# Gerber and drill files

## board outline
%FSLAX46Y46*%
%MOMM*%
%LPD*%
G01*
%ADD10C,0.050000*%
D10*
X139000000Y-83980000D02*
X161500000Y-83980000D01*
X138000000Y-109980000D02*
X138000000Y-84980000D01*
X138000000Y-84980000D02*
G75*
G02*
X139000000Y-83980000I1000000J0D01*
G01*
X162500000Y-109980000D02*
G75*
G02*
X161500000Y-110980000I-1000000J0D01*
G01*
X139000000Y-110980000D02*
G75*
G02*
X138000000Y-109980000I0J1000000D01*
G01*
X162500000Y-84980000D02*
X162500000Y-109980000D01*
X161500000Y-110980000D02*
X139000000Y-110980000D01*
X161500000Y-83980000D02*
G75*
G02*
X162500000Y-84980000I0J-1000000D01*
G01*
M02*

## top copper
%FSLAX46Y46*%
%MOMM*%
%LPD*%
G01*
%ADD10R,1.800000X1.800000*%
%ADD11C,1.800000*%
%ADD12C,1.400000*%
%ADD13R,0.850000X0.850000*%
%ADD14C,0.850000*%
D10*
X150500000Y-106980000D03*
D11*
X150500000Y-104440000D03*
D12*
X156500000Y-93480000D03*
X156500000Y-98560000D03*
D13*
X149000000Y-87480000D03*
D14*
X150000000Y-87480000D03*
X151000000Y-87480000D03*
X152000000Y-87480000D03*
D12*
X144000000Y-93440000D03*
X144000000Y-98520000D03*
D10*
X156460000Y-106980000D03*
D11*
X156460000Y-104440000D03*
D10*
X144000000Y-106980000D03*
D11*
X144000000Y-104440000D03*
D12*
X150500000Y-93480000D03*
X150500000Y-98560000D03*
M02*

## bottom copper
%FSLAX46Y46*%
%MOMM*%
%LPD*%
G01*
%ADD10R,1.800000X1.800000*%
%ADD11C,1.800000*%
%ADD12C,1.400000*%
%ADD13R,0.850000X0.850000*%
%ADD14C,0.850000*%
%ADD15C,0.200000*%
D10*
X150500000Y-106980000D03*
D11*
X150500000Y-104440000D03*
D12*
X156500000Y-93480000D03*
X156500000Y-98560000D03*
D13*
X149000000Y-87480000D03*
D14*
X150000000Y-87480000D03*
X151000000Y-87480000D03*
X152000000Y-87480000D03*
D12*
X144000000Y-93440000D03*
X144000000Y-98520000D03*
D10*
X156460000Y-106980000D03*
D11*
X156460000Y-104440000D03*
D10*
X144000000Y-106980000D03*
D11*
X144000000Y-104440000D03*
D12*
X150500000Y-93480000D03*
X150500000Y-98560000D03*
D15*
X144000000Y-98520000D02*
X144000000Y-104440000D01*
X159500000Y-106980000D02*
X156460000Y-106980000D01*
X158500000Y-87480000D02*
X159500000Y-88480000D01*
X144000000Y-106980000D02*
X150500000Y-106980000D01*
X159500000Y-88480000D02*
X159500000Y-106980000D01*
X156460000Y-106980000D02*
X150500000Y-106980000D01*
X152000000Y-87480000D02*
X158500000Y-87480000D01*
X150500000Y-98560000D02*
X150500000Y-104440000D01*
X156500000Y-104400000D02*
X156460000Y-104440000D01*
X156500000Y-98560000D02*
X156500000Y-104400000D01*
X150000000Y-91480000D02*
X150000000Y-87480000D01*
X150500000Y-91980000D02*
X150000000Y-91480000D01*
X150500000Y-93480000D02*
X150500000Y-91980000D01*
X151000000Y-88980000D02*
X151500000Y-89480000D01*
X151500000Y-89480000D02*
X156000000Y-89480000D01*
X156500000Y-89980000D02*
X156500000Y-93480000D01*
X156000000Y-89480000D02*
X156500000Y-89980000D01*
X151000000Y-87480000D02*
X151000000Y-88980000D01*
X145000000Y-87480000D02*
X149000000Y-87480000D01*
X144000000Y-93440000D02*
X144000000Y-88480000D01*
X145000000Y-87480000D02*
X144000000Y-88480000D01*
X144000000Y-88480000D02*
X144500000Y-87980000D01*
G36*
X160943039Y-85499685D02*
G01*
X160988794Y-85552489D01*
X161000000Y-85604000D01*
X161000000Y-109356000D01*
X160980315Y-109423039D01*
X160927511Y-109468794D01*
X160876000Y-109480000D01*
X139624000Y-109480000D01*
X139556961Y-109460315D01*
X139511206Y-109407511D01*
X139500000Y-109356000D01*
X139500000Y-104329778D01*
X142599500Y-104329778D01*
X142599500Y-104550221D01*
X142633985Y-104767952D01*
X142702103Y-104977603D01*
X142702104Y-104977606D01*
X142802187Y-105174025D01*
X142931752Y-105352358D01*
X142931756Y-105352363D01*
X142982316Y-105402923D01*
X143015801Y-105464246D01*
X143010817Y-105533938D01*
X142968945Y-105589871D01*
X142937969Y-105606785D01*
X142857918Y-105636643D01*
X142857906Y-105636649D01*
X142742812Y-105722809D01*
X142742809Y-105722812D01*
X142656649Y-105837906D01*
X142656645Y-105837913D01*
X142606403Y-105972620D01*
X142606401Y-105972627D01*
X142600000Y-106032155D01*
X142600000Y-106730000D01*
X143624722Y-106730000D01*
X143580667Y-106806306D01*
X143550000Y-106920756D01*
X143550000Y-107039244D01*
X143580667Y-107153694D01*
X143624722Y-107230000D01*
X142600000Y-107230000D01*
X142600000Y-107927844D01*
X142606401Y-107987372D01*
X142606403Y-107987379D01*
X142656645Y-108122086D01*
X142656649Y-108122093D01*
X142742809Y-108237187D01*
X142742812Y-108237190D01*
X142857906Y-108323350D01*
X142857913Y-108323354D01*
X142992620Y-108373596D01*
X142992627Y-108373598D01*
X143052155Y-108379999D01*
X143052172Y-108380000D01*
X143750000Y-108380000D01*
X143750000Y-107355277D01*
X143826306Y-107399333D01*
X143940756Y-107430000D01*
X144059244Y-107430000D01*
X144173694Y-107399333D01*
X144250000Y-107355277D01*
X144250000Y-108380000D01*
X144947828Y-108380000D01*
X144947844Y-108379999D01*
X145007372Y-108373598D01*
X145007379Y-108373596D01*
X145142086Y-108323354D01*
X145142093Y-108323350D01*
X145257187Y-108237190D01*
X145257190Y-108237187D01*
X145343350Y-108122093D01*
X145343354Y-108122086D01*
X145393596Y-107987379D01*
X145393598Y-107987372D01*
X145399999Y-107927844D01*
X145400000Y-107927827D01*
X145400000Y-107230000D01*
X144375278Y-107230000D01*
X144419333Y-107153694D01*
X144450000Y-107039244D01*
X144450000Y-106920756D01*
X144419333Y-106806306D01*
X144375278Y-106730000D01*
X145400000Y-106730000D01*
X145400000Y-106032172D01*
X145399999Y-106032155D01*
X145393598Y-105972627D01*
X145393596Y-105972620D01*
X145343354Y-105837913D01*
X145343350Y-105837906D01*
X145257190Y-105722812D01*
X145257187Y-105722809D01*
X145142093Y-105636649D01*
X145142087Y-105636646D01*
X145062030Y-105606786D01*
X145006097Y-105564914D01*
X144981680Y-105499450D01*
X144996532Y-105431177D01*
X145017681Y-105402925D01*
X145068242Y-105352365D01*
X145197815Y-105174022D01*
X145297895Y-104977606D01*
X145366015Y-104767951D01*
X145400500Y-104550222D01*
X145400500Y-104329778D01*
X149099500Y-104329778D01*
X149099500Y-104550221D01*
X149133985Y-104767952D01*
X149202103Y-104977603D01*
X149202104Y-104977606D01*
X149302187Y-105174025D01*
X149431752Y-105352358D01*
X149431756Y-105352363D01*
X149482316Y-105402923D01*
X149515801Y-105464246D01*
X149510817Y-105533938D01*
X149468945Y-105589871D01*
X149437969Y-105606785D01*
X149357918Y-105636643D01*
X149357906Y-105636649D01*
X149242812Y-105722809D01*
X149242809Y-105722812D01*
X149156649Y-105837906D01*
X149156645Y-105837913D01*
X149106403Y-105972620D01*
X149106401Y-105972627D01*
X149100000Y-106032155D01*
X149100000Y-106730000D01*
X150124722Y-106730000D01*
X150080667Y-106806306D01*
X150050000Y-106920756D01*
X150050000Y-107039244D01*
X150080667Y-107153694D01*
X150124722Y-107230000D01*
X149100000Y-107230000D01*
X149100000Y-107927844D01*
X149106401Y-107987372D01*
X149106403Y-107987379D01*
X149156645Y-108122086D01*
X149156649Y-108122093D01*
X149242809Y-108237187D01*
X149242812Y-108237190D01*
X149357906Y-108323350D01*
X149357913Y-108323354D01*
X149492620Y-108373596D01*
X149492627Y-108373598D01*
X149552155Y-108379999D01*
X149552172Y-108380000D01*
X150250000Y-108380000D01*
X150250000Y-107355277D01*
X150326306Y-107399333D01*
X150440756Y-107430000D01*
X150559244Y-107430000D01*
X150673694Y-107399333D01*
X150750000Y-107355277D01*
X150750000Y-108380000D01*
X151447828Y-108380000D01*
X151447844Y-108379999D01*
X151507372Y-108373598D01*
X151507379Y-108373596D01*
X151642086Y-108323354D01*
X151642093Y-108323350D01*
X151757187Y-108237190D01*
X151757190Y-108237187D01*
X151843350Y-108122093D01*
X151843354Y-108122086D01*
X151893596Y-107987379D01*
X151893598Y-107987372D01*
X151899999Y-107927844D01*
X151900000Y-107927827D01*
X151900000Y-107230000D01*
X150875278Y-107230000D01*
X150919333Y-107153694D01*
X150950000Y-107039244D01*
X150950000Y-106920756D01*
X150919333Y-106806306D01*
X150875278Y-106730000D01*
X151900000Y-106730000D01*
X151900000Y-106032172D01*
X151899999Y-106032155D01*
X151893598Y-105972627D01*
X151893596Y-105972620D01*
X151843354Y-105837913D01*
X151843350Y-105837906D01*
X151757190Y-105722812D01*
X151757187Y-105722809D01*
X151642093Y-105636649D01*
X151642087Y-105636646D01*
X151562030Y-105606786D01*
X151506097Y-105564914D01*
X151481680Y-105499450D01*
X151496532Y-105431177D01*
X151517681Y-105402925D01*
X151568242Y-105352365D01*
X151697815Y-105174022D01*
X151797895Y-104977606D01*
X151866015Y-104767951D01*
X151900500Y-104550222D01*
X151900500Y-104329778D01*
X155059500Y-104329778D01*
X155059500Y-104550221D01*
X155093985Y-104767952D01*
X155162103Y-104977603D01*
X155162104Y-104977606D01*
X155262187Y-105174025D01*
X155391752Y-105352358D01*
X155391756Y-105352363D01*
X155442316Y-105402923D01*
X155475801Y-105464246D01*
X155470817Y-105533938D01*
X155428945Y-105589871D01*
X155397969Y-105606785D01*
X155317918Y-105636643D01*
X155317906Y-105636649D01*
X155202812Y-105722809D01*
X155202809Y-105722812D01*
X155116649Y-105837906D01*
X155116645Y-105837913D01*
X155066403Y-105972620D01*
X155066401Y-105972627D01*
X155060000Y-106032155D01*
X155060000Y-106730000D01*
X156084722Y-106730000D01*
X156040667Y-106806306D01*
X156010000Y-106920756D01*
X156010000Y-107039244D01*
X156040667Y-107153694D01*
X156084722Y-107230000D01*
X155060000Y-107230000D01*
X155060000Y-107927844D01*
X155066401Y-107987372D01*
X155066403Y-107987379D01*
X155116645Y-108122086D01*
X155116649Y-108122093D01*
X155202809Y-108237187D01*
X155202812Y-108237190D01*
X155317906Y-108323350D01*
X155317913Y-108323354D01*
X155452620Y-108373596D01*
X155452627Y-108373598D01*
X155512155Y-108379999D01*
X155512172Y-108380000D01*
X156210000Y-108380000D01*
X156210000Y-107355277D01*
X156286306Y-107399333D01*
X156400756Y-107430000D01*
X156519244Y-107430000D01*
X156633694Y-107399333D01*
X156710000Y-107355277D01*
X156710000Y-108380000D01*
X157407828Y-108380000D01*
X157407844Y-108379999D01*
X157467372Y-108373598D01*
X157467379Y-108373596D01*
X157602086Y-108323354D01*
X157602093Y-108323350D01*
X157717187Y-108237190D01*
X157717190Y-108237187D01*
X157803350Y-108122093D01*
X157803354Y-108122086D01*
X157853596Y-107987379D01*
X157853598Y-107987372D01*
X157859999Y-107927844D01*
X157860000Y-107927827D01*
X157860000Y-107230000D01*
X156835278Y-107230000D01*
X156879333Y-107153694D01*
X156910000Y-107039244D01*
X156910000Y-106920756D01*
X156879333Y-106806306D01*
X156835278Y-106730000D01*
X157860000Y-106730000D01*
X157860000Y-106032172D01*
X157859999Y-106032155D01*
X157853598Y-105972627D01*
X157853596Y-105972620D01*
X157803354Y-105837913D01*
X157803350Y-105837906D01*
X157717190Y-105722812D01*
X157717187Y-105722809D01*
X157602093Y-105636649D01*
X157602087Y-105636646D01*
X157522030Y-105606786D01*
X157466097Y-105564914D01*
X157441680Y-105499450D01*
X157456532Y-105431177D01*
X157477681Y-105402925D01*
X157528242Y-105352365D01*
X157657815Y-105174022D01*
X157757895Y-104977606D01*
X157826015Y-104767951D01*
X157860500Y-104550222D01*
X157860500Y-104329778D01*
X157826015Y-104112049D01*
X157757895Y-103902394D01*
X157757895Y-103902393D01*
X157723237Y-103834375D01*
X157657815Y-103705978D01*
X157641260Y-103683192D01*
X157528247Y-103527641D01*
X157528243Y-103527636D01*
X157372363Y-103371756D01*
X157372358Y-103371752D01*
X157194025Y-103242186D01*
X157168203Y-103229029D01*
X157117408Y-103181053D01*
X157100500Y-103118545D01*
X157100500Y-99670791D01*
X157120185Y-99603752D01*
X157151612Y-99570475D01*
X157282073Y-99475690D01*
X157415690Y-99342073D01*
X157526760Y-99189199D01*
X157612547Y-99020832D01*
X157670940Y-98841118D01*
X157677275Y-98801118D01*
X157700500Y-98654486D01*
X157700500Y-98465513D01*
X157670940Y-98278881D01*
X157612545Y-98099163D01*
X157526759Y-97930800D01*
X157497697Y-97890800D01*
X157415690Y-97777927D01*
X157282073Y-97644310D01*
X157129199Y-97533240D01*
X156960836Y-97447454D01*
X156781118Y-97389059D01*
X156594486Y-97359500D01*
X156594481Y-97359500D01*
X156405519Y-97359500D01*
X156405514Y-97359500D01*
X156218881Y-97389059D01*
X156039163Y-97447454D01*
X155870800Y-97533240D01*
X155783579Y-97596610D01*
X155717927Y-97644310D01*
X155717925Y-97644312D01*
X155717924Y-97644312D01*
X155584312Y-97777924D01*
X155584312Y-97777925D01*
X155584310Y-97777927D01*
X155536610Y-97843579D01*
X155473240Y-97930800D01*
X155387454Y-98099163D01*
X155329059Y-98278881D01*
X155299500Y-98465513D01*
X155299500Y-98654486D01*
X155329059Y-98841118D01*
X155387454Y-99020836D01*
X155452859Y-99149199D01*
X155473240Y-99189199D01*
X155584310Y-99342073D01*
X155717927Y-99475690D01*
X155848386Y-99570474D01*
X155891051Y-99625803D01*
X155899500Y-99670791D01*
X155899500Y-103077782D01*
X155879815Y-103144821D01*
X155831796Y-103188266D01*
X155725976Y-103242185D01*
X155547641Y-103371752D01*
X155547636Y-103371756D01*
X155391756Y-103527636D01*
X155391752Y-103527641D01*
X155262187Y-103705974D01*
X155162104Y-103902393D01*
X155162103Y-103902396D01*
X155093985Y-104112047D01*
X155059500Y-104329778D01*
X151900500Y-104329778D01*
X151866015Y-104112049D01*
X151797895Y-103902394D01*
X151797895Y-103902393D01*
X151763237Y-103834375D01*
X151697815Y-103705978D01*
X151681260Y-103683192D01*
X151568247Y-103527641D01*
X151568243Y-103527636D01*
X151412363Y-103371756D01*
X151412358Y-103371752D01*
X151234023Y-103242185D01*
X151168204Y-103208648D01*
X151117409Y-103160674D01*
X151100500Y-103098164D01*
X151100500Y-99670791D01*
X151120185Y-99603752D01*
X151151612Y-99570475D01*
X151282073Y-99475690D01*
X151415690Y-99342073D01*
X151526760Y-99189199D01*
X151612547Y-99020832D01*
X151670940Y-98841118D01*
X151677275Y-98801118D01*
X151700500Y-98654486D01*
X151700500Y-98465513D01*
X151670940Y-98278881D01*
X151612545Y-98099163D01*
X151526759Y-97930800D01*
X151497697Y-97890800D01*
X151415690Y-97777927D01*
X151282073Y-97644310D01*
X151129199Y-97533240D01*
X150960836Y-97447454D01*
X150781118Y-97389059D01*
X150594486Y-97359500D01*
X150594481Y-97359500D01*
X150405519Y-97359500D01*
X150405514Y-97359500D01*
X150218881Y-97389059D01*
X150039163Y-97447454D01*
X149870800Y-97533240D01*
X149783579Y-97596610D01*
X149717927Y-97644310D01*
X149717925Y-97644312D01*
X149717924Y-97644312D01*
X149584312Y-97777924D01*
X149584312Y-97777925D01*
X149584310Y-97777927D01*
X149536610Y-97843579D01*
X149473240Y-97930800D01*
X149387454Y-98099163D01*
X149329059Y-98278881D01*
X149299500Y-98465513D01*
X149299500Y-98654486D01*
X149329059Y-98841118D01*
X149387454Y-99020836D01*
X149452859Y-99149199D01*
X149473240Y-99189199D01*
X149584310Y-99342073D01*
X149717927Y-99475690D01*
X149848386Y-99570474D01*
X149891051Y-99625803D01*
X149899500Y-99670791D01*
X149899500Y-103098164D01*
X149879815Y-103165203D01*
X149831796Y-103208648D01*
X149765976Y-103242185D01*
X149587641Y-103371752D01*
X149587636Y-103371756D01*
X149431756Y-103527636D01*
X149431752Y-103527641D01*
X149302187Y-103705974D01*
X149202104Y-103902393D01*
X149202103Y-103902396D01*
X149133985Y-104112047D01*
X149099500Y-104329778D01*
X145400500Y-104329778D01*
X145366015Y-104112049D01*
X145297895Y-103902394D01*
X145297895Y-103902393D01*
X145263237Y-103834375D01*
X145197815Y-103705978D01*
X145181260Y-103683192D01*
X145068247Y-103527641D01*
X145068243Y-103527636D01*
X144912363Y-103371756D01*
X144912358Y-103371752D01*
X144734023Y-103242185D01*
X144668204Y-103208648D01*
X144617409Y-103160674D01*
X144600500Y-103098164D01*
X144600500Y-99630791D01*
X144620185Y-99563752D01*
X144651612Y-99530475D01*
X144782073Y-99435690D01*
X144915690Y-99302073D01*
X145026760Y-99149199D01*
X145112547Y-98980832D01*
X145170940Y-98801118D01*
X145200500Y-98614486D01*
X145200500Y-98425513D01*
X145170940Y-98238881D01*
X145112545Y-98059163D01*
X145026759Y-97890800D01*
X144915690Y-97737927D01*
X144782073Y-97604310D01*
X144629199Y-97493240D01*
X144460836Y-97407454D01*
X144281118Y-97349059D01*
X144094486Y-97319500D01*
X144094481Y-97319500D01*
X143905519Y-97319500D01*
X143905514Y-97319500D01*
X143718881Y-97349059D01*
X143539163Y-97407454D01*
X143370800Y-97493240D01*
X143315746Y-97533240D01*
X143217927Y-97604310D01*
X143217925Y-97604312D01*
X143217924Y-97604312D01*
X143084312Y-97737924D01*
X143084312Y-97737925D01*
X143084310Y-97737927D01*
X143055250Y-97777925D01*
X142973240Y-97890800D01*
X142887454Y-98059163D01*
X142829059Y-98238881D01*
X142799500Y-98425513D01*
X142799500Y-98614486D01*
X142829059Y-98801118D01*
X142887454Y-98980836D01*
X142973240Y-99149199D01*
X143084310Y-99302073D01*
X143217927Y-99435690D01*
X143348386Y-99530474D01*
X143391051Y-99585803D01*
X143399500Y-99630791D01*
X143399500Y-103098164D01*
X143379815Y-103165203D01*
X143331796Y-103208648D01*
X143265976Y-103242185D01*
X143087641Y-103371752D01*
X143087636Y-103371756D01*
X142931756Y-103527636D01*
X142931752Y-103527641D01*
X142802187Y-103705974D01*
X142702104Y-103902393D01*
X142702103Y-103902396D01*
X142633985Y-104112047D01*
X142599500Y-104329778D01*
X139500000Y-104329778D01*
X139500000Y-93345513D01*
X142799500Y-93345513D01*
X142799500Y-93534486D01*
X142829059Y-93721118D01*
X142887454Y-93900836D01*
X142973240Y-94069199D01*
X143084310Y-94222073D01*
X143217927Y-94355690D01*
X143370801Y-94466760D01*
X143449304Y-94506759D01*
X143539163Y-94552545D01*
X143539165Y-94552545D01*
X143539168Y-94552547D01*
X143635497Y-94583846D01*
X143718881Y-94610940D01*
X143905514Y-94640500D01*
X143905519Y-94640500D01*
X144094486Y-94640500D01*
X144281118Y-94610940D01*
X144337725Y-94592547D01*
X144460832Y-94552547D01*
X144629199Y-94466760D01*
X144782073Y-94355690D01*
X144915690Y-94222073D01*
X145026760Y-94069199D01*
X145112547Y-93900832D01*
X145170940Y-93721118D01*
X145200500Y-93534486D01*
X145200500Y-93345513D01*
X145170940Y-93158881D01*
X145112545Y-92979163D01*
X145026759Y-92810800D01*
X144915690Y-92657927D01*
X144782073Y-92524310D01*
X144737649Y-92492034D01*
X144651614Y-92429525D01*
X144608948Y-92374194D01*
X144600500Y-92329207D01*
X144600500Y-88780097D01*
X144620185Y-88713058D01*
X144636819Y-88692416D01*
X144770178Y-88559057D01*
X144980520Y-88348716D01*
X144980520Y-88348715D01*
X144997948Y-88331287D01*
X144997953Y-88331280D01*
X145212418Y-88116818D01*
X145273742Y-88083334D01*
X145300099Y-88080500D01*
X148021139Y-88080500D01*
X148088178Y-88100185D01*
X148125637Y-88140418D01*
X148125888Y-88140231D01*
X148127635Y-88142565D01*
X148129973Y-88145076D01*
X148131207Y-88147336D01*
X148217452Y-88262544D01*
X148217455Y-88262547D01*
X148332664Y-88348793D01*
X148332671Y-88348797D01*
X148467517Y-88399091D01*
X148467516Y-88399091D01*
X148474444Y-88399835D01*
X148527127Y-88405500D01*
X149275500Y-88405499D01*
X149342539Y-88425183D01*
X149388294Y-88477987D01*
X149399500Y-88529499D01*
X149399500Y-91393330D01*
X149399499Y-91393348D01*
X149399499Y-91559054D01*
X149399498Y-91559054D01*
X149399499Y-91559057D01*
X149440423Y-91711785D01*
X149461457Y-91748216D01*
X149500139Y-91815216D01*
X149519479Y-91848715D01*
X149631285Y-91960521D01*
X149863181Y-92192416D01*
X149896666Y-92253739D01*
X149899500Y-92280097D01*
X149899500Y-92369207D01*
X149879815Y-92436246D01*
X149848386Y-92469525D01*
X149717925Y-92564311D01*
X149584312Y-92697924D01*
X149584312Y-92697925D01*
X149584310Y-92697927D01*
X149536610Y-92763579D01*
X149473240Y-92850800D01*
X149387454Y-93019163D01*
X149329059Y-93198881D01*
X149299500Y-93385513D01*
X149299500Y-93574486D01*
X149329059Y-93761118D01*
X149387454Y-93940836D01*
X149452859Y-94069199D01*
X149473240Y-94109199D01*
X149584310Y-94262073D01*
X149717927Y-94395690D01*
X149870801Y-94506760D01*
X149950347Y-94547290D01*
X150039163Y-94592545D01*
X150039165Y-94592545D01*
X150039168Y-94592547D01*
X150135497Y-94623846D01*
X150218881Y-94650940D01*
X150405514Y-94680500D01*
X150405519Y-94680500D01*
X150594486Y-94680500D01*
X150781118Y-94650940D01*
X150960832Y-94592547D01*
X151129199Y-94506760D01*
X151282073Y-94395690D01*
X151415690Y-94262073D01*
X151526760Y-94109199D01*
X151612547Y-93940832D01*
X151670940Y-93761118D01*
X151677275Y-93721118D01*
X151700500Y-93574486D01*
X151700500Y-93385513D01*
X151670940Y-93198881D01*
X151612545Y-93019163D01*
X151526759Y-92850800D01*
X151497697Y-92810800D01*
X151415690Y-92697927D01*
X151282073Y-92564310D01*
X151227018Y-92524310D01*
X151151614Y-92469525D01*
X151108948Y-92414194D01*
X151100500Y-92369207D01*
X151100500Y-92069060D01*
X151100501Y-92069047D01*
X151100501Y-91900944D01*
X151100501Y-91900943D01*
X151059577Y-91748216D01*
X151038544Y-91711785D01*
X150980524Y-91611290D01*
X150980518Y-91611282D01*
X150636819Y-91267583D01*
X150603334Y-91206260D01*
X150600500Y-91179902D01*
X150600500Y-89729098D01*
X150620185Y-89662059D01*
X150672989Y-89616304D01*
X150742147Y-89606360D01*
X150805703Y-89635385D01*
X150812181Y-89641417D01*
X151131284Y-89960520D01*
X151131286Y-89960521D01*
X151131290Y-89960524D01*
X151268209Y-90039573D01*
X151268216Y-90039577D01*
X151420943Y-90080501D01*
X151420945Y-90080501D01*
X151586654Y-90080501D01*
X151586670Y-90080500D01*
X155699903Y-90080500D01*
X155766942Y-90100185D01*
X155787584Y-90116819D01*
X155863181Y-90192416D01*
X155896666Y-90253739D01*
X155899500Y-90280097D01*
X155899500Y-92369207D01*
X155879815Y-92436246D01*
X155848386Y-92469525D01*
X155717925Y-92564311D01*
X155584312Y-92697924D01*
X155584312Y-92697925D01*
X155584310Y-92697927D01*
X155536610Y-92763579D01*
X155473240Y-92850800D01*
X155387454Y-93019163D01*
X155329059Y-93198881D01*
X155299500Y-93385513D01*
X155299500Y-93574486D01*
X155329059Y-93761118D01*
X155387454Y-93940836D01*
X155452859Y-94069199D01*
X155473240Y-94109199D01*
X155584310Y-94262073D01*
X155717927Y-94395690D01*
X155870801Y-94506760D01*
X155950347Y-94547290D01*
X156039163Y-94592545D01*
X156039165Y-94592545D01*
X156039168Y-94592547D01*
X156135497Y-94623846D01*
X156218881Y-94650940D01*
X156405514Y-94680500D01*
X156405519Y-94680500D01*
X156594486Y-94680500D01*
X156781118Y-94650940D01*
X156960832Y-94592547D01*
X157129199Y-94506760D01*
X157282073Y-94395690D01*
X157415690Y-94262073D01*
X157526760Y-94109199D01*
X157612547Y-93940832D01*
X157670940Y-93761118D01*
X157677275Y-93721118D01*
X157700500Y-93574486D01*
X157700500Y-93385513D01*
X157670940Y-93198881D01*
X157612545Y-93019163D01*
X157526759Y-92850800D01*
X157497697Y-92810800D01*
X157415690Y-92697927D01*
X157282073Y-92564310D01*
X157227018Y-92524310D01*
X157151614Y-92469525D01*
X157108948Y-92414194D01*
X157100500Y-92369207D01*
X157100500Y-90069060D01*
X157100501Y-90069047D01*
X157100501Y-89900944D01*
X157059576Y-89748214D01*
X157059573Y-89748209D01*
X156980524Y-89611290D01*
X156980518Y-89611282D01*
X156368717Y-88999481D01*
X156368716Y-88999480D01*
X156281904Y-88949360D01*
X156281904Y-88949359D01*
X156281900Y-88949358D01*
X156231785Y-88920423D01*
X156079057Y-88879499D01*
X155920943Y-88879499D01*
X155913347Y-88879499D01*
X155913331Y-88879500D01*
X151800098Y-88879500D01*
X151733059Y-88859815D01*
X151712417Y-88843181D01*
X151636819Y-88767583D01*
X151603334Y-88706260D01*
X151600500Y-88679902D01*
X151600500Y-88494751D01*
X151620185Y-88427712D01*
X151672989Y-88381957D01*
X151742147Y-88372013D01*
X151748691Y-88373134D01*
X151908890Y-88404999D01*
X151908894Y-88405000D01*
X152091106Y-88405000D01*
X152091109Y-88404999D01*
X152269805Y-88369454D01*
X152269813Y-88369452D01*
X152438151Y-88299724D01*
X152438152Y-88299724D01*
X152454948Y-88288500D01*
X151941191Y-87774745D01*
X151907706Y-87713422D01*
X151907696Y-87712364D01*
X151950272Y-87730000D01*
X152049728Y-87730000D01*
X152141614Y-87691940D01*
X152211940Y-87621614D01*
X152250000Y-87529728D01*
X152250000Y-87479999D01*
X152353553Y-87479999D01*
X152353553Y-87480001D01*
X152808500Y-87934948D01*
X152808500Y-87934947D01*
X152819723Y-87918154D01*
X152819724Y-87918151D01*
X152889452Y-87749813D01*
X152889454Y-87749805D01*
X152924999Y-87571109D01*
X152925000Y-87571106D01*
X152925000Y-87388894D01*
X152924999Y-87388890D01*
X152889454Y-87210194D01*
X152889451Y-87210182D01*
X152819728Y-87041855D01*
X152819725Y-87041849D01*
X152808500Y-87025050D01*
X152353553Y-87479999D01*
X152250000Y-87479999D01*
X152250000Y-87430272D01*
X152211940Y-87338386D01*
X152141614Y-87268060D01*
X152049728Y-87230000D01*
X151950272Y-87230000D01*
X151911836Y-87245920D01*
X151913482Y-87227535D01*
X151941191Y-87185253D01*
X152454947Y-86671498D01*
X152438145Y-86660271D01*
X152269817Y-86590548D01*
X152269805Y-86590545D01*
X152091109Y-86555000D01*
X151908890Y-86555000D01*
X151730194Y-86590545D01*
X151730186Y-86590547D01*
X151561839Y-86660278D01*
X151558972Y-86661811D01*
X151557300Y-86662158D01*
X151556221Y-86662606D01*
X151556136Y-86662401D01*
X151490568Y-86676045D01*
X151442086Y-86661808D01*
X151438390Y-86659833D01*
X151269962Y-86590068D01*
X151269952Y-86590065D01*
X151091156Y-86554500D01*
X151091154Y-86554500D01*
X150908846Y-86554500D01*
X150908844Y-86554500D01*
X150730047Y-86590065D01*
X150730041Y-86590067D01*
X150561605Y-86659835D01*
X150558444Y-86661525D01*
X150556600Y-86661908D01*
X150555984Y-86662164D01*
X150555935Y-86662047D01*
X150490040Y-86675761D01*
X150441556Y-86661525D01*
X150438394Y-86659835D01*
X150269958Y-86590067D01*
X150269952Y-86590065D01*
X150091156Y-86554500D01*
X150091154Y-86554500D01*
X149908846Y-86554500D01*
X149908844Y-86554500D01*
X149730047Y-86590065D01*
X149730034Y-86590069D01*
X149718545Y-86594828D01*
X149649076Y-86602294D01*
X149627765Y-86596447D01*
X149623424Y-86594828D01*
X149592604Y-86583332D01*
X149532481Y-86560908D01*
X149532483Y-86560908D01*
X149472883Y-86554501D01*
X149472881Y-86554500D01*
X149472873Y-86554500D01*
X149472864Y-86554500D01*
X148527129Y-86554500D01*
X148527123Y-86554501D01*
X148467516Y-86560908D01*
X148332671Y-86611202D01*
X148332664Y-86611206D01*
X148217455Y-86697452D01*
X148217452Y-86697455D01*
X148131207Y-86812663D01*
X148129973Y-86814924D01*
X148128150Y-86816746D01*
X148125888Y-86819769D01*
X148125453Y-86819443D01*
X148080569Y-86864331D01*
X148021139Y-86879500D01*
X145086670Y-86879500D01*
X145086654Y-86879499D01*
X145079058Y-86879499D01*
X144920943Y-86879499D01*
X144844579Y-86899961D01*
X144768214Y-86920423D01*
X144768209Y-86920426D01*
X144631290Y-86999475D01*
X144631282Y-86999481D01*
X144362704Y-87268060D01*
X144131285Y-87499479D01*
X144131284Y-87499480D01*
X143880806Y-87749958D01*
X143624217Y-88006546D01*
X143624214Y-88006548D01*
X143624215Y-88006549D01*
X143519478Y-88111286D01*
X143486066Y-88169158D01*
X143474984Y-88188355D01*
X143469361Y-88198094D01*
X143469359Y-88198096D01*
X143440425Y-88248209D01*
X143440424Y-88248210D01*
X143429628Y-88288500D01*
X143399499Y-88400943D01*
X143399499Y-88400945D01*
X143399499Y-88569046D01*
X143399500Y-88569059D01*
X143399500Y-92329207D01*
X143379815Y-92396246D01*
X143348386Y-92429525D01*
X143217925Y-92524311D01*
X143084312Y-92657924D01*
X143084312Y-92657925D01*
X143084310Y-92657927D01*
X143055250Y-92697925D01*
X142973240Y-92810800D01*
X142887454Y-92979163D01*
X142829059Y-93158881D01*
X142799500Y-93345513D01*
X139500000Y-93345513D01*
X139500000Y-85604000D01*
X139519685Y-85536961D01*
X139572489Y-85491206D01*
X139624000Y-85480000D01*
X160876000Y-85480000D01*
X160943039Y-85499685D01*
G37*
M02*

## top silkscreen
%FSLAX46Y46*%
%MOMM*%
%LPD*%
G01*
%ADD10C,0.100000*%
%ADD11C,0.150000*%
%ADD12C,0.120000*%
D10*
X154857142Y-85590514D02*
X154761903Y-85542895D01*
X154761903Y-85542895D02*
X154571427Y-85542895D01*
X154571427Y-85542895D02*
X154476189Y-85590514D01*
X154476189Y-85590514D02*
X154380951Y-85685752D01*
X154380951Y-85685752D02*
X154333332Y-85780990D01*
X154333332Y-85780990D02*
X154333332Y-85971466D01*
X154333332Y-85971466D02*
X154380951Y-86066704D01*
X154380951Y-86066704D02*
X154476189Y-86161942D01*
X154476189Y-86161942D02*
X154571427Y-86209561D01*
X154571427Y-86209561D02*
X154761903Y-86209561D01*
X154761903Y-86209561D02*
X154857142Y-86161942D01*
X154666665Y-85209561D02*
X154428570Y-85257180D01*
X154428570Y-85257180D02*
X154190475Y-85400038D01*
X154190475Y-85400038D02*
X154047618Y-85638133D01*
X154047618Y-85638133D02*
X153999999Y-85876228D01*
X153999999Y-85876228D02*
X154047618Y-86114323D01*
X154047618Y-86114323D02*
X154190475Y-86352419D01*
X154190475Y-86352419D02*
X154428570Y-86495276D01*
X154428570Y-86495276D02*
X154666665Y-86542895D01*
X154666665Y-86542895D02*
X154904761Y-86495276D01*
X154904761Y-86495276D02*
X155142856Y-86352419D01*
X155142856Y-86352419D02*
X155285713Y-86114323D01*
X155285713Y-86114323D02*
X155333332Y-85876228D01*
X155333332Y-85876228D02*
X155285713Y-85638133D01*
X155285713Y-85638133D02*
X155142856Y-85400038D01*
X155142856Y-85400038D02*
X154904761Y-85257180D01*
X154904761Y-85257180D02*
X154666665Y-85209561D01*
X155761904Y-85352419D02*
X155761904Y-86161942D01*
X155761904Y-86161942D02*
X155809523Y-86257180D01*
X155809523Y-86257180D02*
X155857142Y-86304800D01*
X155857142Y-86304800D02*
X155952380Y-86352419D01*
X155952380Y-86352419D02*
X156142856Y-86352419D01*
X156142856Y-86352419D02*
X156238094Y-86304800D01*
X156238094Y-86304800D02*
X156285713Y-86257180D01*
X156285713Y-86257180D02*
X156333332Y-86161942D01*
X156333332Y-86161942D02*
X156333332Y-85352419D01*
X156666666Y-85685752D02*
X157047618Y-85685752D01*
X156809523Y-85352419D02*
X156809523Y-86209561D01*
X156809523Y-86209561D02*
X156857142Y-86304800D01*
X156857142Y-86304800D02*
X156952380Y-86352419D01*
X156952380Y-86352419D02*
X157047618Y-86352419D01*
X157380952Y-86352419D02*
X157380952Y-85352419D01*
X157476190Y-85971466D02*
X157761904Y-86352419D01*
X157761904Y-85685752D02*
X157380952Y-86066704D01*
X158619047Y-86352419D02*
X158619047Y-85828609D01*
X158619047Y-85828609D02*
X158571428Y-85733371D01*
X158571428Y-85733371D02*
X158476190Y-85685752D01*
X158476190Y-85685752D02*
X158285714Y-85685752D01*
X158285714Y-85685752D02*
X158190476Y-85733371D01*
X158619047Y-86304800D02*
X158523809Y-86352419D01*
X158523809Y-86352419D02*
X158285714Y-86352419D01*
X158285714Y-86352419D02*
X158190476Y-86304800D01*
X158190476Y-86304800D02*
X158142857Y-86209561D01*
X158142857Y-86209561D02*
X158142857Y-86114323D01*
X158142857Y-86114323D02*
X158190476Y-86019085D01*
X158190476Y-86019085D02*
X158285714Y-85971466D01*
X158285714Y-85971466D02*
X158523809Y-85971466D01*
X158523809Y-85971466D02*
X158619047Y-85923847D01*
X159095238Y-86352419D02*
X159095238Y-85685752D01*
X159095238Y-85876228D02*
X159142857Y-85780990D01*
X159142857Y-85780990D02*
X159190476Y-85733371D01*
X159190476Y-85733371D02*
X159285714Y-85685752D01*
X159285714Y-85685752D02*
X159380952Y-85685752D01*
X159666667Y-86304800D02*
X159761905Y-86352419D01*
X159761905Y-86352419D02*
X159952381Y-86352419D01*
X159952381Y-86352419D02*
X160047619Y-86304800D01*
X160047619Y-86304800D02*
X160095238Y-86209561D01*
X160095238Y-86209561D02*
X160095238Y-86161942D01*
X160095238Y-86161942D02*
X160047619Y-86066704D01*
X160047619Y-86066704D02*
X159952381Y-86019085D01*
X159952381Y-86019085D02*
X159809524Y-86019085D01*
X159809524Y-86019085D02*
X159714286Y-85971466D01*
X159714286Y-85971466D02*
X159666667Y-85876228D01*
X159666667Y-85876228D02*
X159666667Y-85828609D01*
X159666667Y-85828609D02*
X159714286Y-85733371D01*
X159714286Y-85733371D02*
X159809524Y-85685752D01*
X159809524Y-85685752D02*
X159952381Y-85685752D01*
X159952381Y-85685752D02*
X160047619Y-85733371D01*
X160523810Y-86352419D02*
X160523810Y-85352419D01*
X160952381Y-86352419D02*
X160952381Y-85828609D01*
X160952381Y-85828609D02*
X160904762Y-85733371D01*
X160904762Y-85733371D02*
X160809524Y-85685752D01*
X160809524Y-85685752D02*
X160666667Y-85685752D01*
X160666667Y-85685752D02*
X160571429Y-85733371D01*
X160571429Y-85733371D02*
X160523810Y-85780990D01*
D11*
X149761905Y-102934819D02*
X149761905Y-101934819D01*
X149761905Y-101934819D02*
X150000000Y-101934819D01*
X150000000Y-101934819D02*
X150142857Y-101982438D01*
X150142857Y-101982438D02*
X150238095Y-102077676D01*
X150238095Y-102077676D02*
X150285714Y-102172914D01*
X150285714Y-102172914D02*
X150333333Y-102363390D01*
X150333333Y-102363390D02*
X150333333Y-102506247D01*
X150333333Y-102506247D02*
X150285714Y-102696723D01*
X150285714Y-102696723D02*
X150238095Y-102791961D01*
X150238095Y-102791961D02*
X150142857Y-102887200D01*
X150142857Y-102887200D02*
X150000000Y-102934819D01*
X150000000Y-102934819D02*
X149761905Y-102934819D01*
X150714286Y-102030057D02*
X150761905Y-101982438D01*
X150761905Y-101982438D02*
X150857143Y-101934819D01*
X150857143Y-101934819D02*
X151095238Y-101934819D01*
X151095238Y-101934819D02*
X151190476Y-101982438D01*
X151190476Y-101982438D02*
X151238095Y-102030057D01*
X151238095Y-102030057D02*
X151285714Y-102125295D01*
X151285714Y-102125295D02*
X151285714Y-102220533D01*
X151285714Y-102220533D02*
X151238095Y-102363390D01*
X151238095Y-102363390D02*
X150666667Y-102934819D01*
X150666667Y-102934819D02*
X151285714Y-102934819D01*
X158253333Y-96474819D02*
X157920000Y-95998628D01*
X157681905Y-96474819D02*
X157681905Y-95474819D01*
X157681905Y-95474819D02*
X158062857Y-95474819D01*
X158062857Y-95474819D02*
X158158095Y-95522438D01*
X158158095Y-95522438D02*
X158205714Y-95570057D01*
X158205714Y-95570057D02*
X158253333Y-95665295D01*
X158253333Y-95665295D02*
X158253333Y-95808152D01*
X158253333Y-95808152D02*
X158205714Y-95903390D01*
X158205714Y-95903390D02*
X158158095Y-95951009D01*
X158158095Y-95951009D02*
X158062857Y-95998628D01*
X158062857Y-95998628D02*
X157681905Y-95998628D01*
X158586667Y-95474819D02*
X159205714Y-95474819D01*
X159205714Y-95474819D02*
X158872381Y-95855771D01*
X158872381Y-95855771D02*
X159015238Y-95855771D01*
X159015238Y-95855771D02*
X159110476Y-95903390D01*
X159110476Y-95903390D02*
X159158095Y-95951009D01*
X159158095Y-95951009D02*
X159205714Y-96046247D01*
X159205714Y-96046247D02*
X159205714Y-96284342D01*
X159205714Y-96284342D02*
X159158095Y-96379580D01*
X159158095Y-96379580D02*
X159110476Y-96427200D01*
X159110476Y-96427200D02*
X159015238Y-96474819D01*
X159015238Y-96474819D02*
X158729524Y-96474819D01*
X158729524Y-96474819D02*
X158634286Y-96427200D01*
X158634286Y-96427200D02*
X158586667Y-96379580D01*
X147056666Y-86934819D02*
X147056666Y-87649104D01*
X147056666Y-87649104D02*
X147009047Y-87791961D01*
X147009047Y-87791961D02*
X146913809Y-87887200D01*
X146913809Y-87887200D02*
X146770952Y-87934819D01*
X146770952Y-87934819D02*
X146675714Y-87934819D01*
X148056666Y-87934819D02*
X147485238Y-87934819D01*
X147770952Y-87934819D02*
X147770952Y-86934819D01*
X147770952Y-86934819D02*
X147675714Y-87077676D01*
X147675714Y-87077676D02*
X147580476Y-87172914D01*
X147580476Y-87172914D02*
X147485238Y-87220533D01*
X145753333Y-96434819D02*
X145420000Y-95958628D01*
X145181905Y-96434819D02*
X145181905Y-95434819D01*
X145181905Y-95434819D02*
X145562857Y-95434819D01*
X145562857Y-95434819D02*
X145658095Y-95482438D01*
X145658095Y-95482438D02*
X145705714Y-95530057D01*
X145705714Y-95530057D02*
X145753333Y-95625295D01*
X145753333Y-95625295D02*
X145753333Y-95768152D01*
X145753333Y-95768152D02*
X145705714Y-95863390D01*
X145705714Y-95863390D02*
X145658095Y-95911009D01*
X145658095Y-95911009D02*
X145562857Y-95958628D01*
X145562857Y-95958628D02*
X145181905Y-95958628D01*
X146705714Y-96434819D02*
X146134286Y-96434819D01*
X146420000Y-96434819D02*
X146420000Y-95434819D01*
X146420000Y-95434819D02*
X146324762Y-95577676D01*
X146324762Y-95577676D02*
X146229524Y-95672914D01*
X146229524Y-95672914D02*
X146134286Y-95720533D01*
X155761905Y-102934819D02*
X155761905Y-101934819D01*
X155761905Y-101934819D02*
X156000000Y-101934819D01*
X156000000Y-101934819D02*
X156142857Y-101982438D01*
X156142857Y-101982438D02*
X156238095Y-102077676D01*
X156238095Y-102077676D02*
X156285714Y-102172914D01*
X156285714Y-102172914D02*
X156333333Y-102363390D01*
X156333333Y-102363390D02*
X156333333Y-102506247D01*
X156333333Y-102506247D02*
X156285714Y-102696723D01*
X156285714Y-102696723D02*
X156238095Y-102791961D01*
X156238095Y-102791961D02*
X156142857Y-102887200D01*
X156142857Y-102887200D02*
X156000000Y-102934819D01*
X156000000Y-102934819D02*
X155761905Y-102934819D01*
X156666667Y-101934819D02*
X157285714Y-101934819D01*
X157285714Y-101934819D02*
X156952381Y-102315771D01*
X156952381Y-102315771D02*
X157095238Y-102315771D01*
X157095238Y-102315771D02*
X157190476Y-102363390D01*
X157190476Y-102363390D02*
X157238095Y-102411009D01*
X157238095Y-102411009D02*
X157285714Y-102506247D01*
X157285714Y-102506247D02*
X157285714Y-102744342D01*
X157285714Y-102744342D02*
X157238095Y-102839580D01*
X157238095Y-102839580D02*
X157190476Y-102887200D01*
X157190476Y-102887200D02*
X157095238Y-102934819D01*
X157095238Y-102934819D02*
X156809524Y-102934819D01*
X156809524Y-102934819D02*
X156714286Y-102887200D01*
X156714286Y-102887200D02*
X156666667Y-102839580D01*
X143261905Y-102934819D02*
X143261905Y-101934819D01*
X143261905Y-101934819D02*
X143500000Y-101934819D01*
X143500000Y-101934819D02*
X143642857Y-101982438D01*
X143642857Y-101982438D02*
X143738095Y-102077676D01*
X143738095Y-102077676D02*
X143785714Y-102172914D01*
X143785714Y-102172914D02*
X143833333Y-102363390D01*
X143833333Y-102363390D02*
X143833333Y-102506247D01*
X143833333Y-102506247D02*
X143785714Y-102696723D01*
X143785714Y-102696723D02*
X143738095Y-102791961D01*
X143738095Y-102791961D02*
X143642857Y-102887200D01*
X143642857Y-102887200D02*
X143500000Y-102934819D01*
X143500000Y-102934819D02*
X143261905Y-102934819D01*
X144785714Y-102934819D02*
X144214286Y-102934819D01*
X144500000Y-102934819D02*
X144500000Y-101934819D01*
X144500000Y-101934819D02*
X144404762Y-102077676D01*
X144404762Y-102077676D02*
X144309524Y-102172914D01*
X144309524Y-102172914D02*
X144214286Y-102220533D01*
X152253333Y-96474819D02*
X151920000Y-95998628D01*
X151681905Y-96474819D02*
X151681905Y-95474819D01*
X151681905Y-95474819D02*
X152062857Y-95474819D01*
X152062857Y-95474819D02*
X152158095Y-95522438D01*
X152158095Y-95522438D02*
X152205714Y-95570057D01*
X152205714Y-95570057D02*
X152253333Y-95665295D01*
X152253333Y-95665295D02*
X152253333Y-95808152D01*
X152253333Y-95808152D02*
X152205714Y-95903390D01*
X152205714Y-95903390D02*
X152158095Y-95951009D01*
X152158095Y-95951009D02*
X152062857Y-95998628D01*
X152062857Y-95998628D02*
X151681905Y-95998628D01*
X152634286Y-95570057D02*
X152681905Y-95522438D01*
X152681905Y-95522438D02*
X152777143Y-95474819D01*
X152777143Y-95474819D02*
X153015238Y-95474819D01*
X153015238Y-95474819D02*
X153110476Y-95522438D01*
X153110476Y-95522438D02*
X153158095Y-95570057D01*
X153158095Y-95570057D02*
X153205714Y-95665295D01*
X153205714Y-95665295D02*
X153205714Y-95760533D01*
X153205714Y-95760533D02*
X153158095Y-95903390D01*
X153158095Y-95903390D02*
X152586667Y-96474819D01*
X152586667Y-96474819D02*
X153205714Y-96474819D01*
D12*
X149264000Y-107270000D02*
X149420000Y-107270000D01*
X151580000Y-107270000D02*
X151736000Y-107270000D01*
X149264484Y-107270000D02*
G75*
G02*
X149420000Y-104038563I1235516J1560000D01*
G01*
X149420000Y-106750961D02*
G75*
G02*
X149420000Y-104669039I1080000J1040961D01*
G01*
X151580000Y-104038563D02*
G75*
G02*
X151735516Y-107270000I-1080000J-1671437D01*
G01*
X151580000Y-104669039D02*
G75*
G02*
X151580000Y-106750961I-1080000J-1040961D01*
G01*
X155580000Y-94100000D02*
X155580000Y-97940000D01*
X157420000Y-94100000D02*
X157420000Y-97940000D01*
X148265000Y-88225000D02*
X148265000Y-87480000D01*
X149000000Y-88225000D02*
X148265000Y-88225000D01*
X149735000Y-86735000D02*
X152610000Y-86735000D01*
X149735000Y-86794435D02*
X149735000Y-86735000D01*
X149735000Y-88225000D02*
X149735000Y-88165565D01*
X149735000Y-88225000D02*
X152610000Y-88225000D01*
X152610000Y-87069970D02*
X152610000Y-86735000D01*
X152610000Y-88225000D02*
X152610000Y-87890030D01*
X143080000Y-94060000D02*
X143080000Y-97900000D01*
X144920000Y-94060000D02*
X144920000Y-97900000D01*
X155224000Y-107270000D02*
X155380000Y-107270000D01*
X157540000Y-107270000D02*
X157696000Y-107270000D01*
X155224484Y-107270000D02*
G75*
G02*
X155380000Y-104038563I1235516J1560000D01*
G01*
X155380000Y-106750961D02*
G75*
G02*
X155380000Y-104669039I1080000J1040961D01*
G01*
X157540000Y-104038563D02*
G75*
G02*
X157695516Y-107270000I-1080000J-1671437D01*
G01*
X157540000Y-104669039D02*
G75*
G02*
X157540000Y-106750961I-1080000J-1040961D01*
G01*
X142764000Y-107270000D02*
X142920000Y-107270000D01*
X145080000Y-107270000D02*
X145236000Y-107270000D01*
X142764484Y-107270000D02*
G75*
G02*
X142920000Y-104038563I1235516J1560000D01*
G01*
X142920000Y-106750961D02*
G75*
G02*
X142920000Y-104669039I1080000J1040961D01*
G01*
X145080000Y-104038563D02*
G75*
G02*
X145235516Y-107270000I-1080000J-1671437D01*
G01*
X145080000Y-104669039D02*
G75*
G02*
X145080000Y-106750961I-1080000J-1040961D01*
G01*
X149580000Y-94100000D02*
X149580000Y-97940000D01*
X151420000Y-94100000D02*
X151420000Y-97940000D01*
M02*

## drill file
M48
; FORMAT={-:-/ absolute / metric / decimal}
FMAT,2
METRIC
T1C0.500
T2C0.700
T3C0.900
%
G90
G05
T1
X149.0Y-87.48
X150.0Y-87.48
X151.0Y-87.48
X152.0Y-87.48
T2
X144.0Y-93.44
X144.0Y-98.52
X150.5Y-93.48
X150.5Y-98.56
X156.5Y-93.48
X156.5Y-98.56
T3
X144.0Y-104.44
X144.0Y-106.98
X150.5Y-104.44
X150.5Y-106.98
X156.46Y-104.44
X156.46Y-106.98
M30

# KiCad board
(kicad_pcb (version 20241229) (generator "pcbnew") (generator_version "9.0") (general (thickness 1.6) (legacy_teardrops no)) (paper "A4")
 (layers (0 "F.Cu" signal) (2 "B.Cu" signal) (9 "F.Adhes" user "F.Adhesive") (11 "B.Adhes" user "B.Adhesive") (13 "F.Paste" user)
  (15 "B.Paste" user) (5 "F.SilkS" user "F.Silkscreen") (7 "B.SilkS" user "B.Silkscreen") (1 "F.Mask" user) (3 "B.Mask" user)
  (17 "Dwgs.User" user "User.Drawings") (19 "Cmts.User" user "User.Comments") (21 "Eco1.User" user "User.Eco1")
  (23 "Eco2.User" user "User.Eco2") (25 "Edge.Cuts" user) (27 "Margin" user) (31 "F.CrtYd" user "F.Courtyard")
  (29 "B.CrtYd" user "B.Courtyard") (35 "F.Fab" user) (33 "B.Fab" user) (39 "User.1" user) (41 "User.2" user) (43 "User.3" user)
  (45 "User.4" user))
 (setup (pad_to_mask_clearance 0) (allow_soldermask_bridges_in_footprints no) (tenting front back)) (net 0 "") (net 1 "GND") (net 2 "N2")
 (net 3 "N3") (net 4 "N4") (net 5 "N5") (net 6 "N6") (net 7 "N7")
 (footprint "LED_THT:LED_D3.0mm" (layer "F.Cu") (at 150.5 106.98 90)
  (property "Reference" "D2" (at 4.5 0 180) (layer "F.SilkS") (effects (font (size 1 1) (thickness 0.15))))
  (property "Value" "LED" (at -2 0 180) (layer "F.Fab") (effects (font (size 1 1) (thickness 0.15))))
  (fp_line (start -0.29 -1.236) (end -0.29 -1.08) (stroke (width 0.12) (type solid)) (layer "F.SilkS"))
  (fp_line (start -0.29 1.08) (end -0.29 1.236) (stroke (width 0.12) (type solid)) (layer "F.SilkS"))
  (fp_arc (start -0.29 -1.235516) (mid 1.36566 -1.987699) (end 2.941437 -1.08) (stroke (width 0.12) (type solid)) (layer "F.SilkS"))
  (fp_arc (start 0.229039 -1.08) (mid 1.27 -1.5) (end 2.310961 -1.08) (stroke (width 0.12) (type solid)) (layer "F.SilkS"))
  (fp_arc (start 2.941437 1.08) (mid 1.36566 1.987699) (end -0.29 1.235516) (stroke (width 0.12) (type solid)) (layer "F.SilkS"))
  (fp_arc (start 2.310961 1.08) (mid 1.27 1.5) (end 0.229039 1.08) (stroke (width 0.12) (type solid)) (layer "F.SilkS"))
  (pad "1" thru_hole rect (at 0 0 90) (size 1.8 1.8) (drill 0.9) (layers "*.Cu" "*.Mask") (remove_unused_layers no) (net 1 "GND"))
  (pad "2" thru_hole circle (at 2.54 0 90) (size 1.8 1.8) (drill 0.9) (layers "*.Cu" "*.Mask") (remove_unused_layers no) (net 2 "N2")))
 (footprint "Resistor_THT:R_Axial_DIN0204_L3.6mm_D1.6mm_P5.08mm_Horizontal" (layer "F.Cu") (at 156.5 93.48 -90)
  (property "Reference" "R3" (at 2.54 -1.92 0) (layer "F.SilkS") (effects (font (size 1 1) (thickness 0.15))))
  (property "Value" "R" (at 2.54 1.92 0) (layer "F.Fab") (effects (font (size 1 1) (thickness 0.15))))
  (fp_line (start 0.62 0.92) (end 4.46 0.92) (stroke (width 0.12) (type solid)) (layer "F.SilkS"))
  (fp_line (start 0.62 -0.92) (end 4.46 -0.92) (stroke (width 0.12) (type solid)) (layer "F.SilkS"))
  (pad "1" thru_hole circle (at 0 0 270) (size 1.4 1.4) (drill 0.7) (layers "*.Cu" "*.Mask") (remove_unused_layers no) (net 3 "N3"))
  (pad "2" thru_hole circle (at 5.08 0 270) (size 1.4 1.4) (drill 0.7) (layers "*.Cu" "*.Mask") (remove_unused_layers no) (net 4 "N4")))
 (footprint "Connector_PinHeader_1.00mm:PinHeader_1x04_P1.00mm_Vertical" (layer "F.Cu") (at 149 87.48 90)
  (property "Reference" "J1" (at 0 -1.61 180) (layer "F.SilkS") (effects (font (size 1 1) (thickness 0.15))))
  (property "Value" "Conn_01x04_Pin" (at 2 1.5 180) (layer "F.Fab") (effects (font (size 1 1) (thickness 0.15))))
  (fp_line (start -0.745 -0.735) (end 0 -0.735) (stroke (width 0.12) (type solid)) (layer "F.SilkS"))
  (fp_line (start -0.745 0) (end -0.745 -0.735) (stroke (width 0.12) (type solid)) (layer "F.SilkS"))
  (fp_line (start 0.745 0.735) (end 0.745 3.61) (stroke (width 0.12) (type solid)) (layer "F.SilkS"))
  (fp_line (start 0.685565 0.735) (end 0.745 0.735) (stroke (width 0.12) (type solid)) (layer "F.SilkS"))
  (fp_line (start -0.745 0.735) (end -0.685565 0.735) (stroke (width 0.12) (type solid)) (layer "F.SilkS"))
  (fp_line (start -0.745 0.735) (end -0.745 3.61) (stroke (width 0.12) (type solid)) (layer "F.SilkS"))
  (fp_line (start 0.41003 3.61) (end 0.745 3.61) (stroke (width 0.12) (type solid)) (layer "F.SilkS"))
  (fp_line (start -0.745 3.61) (end -0.41003 3.61) (stroke (width 0.12) (type solid)) (layer "F.SilkS"))
  (pad "1" thru_hole rect (at 0 0 90) (size 0.85 0.85) (drill 0.5) (layers "*.Cu" "*.Mask") (remove_unused_layers no) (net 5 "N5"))
  (pad "2" thru_hole circle (at 0 1 90) (size 0.85 0.85) (drill 0.5) (layers "*.Cu" "*.Mask") (remove_unused_layers no) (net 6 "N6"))
  (pad "3" thru_hole circle (at 0 2 90) (size 0.85 0.85) (drill 0.5) (layers "*.Cu" "*.Mask") (remove_unused_layers no) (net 3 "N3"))
  (pad "4" thru_hole circle (at 0 3 90) (size 0.85 0.85) (drill 0.5) (layers "*.Cu" "*.Mask") (remove_unused_layers no) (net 1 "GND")))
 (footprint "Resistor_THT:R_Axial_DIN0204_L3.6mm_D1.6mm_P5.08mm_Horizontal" (layer "F.Cu") (at 144 93.44 -90)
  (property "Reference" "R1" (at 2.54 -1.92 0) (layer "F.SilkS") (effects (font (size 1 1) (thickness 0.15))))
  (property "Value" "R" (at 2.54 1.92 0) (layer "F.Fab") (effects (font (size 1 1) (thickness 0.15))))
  (fp_line (start 0.62 0.92) (end 4.46 0.92) (stroke (width 0.12) (type solid)) (layer "F.SilkS"))
  (fp_line (start 0.62 -0.92) (end 4.46 -0.92) (stroke (width 0.12) (type solid)) (layer "F.SilkS"))
  (pad "1" thru_hole circle (at 0 0 270) (size 1.4 1.4) (drill 0.7) (layers "*.Cu" "*.Mask") (remove_unused_layers no) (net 5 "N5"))
  (pad "2" thru_hole circle (at 5.08 0 270) (size 1.4 1.4) (drill 0.7) (layers "*.Cu" "*.Mask") (remove_unused_layers no) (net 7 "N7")))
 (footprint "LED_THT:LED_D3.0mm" (layer "F.Cu") (at 156.46 106.98 90)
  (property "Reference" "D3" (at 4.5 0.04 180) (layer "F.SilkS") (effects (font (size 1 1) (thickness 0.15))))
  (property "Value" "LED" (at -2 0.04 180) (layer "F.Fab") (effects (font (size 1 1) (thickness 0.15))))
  (fp_line (start -0.29 -1.236) (end -0.29 -1.08) (stroke (width 0.12) (type solid)) (layer "F.SilkS"))
  (fp_line (start -0.29 1.08) (end -0.29 1.236) (stroke (width 0.12) (type solid)) (layer "F.SilkS"))
  (fp_arc (start -0.29 -1.235516) (mid 1.36566 -1.987699) (end 2.941437 -1.08) (stroke (width 0.12) (type solid)) (layer "F.SilkS"))
  (fp_arc (start 0.229039 -1.08) (mid 1.27 -1.5) (end 2.310961 -1.08) (stroke (width 0.12) (type solid)) (layer "F.SilkS"))
  (fp_arc (start 2.941437 1.08) (mid 1.36566 1.987699) (end -0.29 1.235516) (stroke (width 0.12) (type solid)) (layer "F.SilkS"))
  (fp_arc (start 2.310961 1.08) (mid 1.27 1.5) (end 0.229039 1.08) (stroke (width 0.12) (type solid)) (layer "F.SilkS"))
  (pad "1" thru_hole rect (at 0 0 90) (size 1.8 1.8) (drill 0.9) (layers "*.Cu" "*.Mask") (remove_unused_layers no) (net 1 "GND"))
  (pad "2" thru_hole circle (at 2.54 0 90) (size 1.8 1.8) (drill 0.9) (layers "*.Cu" "*.Mask") (remove_unused_layers no) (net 4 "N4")))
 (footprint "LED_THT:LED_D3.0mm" (layer "F.Cu") (at 144 106.98 90)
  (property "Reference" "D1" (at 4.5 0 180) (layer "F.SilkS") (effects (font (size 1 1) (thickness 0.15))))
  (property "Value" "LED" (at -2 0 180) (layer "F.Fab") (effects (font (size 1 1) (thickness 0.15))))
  (fp_line (start -0.29 -1.236) (end -0.29 -1.08) (stroke (width 0.12) (type solid)) (layer "F.SilkS"))
  (fp_line (start -0.29 1.08) (end -0.29 1.236) (stroke (width 0.12) (type solid)) (layer "F.SilkS"))
  (fp_arc (start -0.29 -1.235516) (mid 1.36566 -1.987699) (end 2.941437 -1.08) (stroke (width 0.12) (type solid)) (layer "F.SilkS"))
  (fp_arc (start 0.229039 -1.08) (mid 1.27 -1.5) (end 2.310961 -1.08) (stroke (width 0.12) (type solid)) (layer "F.SilkS"))
  (fp_arc (start 2.941437 1.08) (mid 1.36566 1.987699) (end -0.29 1.235516) (stroke (width 0.12) (type solid)) (layer "F.SilkS"))
  (fp_arc (start 2.310961 1.08) (mid 1.27 1.5) (end 0.229039 1.08) (stroke (width 0.12) (type solid)) (layer "F.SilkS"))
  (pad "1" thru_hole rect (at 0 0 90) (size 1.8 1.8) (drill 0.9) (layers "*.Cu" "*.Mask") (remove_unused_layers no) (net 1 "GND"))
  (pad "2" thru_hole circle (at 2.54 0 90) (size 1.8 1.8) (drill 0.9) (layers "*.Cu" "*.Mask") (remove_unused_layers no) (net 7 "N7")))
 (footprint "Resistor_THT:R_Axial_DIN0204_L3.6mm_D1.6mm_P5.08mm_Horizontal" (layer "F.Cu") (at 150.5 93.48 -90)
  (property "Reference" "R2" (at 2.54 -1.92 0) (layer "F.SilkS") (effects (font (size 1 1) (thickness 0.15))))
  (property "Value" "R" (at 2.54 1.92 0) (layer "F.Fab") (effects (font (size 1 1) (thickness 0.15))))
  (fp_line (start 0.62 0.92) (end 4.46 0.92) (stroke (width 0.12) (type solid)) (layer "F.SilkS"))
  (fp_line (start 0.62 -0.92) (end 4.46 -0.92) (stroke (width 0.12) (type solid)) (layer "F.SilkS"))
  (pad "1" thru_hole circle (at 0 0 270) (size 1.4 1.4) (drill 0.7) (layers "*.Cu" "*.Mask") (remove_unused_layers no) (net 6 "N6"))
  (pad "2" thru_hole circle (at 5.08 0 270) (size 1.4 1.4) (drill 0.7) (layers "*.Cu" "*.Mask") (remove_unused_layers no) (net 2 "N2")))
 (gr_line (start 139 83.98) (end 161.5 83.98) (stroke (width 0.05) (type default)) (layer "Edge.Cuts"))
 (gr_line (start 138 109.98) (end 138 84.98) (stroke (width 0.05) (type default)) (layer "Edge.Cuts"))
 (gr_arc (start 138 84.98) (mid 138.292893 84.272893) (end 139 83.98) (stroke (width 0.05) (type default)) (layer "Edge.Cuts"))
 (gr_arc (start 162.5 109.98) (mid 162.207107 110.687107) (end 161.5 110.98) (stroke (width 0.05) (type default)) (layer "Edge.Cuts"))
 (gr_arc (start 139 110.98) (mid 138.292893 110.687107) (end 138 109.98) (stroke (width 0.05) (type default)) (layer "Edge.Cuts"))
 (gr_line (start 162.5 84.98) (end 162.5 109.98) (stroke (width 0.05) (type default)) (layer "Edge.Cuts"))
 (gr_line (start 161.5 110.98) (end 139 110.98) (stroke (width 0.05) (type default)) (layer "Edge.Cuts"))
 (gr_arc (start 161.5 83.98) (mid 162.207107 84.272893) (end 162.5 84.98) (stroke (width 0.05) (type default)) (layer "Edge.Cuts"))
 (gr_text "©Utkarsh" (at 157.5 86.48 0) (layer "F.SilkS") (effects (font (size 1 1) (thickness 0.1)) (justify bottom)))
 (segment (start 144 98.52) (end 144 104.44) (width 0.2) (layer "B.Cu") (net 7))
 (segment (start 159.5 106.98) (end 156.46 106.98) (width 0.2) (layer "B.Cu") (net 1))
 (segment (start 158.5 87.48) (end 159.5 88.48) (width 0.2) (layer "B.Cu") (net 1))
 (segment (start 144 106.98) (end 150.5 106.98) (width 0.2) (layer "B.Cu") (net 1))
 (segment (start 159.5 88.48) (end 159.5 106.98) (width 0.2) (layer "B.Cu") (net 1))
 (segment (start 156.46 106.98) (end 150.5 106.98) (width 0.2) (layer "B.Cu") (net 1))
 (segment (start 152 87.48) (end 158.5 87.48) (width 0.2) (layer "B.Cu") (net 1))
 (segment (start 150.5 98.56) (end 150.5 104.44) (width 0.2) (layer "B.Cu") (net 2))
 (segment (start 156.5 104.4) (end 156.46 104.44) (width 0.2) (layer "B.Cu") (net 4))
 (segment (start 156.5 98.56) (end 156.5 104.4) (width 0.2) (layer "B.Cu") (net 4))
 (segment (start 150 91.48) (end 150 87.48) (width 0.2) (layer "B.Cu") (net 6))
 (segment (start 150.5 91.98) (end 150 91.48) (width 0.2) (layer "B.Cu") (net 6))
 (segment (start 150.5 93.48) (end 150.5 91.98) (width 0.2) (layer "B.Cu") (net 6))
 (segment (start 151 88.98) (end 151.5 89.48) (width 0.2) (layer "B.Cu") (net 3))
 (segment (start 151.5 89.48) (end 156 89.48) (width 0.2) (layer "B.Cu") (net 3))
 (segment (start 156.5 89.98) (end 156.5 93.48) (width 0.2) (layer "B.Cu") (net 3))
 (segment (start 156 89.48) (end 156.5 89.98) (width 0.2) (layer "B.Cu") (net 3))
 (segment (start 151 87.48) (end 151 88.98) (width 0.2) (layer "B.Cu") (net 3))
 (segment (start 145 87.48) (end 149 87.48) (width 0.2) (layer "B.Cu") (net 5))
 (segment (start 144 93.44) (end 144 88.48) (width 0.2) (layer "B.Cu") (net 5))
 (segment (start 145 87.48) (end 144 88.48) (width 0.2) (layer "B.Cu") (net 5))
 (segment (start 144 88.48) (end 144.5 87.98) (width 0.2) (layer "B.Cu") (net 5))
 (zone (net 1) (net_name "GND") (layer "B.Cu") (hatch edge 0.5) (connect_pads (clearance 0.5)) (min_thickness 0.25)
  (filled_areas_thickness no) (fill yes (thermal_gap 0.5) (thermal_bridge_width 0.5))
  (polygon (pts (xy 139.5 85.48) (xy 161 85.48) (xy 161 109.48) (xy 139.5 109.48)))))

